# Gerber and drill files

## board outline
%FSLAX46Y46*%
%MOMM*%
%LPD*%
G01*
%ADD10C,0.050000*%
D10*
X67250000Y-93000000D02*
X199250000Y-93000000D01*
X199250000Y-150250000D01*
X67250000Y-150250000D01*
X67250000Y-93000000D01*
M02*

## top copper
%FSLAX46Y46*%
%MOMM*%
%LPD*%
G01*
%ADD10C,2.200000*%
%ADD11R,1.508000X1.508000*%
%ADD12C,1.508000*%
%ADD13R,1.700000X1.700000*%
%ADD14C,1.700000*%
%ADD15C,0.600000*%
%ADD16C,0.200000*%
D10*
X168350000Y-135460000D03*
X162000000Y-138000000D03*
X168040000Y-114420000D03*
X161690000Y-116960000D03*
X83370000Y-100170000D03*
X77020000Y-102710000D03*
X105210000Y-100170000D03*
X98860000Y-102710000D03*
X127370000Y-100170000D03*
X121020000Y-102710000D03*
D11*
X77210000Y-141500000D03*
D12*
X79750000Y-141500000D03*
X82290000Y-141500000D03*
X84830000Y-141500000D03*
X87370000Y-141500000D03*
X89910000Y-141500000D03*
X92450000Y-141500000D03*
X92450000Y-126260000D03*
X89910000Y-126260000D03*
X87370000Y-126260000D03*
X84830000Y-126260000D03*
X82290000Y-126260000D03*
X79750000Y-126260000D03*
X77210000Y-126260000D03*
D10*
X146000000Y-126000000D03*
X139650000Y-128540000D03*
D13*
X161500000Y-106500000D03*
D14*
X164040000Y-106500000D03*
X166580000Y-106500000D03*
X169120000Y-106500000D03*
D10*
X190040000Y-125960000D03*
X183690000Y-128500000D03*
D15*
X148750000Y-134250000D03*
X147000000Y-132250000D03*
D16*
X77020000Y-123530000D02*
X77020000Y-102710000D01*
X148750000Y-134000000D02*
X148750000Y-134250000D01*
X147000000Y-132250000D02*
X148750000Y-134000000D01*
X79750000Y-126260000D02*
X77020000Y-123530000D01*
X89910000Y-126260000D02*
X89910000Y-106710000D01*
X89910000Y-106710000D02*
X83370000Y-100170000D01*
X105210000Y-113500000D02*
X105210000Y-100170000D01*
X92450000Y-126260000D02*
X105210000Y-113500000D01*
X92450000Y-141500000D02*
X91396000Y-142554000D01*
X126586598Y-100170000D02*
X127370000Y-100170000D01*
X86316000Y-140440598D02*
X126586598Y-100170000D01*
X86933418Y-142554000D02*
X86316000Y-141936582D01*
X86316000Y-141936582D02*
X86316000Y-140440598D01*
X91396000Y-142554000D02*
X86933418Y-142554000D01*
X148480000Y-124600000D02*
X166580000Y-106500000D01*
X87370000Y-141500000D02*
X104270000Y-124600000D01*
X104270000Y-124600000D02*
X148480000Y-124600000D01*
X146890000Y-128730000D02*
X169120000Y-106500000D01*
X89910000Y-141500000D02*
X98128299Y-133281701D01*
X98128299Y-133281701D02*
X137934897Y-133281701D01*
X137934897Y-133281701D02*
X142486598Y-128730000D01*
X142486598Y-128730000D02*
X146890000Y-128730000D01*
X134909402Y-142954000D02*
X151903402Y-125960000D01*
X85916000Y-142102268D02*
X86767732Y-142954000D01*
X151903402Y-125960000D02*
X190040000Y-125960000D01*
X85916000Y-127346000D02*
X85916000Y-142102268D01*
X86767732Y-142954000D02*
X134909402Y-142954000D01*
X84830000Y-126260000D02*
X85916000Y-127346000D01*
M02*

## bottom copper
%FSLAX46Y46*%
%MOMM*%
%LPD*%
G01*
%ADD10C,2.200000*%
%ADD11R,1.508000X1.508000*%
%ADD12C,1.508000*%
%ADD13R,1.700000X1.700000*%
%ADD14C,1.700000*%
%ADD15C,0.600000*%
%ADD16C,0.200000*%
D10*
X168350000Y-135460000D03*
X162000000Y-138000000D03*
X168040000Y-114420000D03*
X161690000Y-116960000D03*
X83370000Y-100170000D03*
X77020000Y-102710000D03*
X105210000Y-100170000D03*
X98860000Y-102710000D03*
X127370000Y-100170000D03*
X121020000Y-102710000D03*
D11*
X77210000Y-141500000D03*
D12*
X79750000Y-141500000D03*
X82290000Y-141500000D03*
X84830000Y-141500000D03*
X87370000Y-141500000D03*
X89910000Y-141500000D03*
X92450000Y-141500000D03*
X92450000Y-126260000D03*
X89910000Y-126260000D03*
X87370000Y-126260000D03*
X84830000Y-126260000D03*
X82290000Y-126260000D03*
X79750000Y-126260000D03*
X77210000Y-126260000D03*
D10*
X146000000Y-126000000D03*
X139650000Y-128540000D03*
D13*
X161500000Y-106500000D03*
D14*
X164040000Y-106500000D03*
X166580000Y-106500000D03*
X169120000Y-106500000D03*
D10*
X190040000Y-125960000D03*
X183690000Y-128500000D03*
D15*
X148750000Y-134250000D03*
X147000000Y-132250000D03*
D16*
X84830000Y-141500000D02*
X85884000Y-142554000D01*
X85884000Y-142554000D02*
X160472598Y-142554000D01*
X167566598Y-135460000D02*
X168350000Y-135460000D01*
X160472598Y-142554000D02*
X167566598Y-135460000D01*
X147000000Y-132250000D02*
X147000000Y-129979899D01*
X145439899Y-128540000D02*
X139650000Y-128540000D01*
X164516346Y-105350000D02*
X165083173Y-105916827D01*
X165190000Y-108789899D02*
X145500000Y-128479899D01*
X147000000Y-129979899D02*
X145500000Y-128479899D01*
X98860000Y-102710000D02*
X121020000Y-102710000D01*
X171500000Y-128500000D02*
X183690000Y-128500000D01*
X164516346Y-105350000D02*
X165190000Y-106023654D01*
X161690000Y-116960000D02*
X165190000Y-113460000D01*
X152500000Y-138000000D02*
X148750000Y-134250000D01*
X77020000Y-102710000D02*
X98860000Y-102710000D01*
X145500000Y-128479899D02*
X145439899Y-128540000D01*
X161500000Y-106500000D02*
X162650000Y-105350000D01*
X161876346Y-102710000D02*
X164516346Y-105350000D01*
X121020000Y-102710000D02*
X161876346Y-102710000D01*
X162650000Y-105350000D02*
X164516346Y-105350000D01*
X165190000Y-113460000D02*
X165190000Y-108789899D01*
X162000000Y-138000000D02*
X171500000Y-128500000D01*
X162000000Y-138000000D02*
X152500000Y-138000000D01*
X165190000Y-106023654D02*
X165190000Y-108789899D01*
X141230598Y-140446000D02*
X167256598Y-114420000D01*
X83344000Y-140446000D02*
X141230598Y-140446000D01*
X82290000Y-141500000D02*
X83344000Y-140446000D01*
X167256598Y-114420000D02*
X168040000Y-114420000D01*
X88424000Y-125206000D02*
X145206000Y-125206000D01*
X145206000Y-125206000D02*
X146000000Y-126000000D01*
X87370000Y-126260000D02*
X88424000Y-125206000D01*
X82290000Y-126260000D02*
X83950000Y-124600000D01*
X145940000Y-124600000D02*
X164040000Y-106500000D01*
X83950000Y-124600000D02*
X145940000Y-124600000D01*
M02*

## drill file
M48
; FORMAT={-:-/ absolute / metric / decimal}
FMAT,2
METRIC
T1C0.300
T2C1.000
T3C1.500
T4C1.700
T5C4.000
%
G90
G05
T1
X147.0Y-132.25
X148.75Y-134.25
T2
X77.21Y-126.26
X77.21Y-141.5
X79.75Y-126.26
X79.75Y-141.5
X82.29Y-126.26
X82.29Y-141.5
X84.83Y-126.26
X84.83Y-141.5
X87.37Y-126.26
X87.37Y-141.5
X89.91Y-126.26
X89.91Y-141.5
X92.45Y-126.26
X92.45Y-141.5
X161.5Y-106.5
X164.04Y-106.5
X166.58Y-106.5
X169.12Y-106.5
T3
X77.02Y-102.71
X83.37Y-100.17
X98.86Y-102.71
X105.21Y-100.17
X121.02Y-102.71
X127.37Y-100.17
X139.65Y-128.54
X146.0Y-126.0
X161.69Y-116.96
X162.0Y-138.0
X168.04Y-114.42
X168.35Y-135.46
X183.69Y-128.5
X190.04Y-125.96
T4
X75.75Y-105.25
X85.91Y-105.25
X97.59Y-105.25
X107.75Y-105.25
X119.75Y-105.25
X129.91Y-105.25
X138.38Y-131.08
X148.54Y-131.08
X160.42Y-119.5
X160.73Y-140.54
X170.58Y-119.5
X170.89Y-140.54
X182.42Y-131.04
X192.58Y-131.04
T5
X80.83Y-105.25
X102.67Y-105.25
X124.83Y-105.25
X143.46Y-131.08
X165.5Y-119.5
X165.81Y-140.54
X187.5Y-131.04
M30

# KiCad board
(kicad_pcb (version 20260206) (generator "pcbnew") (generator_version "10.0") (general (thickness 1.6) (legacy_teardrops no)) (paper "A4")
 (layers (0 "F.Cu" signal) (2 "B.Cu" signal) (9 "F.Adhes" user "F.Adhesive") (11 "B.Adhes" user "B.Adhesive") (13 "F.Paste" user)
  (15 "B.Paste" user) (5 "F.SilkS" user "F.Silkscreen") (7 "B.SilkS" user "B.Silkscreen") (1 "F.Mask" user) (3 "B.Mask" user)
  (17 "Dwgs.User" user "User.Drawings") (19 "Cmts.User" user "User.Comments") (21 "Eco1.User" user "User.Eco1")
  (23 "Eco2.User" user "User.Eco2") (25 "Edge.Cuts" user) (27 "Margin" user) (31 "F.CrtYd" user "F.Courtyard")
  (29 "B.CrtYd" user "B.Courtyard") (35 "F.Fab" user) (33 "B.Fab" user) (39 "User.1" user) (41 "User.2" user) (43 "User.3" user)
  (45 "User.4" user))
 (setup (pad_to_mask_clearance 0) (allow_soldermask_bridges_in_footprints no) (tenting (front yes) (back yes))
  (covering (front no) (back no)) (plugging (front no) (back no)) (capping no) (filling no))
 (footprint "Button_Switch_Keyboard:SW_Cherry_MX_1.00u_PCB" (layer "F.Cu") (at 168.35 135.46)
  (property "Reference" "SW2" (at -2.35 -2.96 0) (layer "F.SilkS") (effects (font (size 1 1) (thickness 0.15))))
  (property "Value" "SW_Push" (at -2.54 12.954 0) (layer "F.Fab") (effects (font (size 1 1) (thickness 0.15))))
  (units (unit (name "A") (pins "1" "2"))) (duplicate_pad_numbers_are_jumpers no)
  (pad "" np_thru_hole circle (at -7.62 5.08) (size 1.7 1.7) (drill 1.7) (layers "*.Cu" "*.Mask"))
  (pad "" np_thru_hole circle (at -2.54 5.08) (size 4 4) (drill 4) (layers "*.Cu" "*.Mask"))
  (pad "" np_thru_hole circle (at 2.54 5.08) (size 1.7 1.7) (drill 1.7) (layers "*.Cu" "*.Mask"))
  (pad "1" thru_hole circle (at 0 0) (size 2.2 2.2) (drill 1.5) (layers "*.Cu" "*.Mask") (remove_unused_layers no) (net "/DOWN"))
  (pad "2" thru_hole circle (at -6.35 2.54) (size 2.2 2.2) (drill 1.5) (layers "*.Cu" "*.Mask") (remove_unused_layers no) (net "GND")))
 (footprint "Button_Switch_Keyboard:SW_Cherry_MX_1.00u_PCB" (layer "F.Cu") (at 168.04 114.42)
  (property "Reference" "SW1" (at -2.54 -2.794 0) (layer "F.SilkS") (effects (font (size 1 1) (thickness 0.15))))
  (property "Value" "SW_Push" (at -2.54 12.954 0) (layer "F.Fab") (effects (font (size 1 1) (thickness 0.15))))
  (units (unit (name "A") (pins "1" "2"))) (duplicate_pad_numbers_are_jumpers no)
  (pad "" np_thru_hole circle (at -7.62 5.08) (size 1.7 1.7) (drill 1.7) (layers "*.Cu" "*.Mask"))
  (pad "" np_thru_hole circle (at -2.54 5.08) (size 4 4) (drill 4) (layers "*.Cu" "*.Mask"))
  (pad "" np_thru_hole circle (at 2.54 5.08) (size 1.7 1.7) (drill 1.7) (layers "*.Cu" "*.Mask"))
  (pad "1" thru_hole circle (at 0 0) (size 2.2 2.2) (drill 1.5) (layers "*.Cu" "*.Mask") (remove_unused_layers no) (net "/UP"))
  (pad "2" thru_hole circle (at -6.35 2.54) (size 2.2 2.2) (drill 1.5) (layers "*.Cu" "*.Mask") (remove_unused_layers no) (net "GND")))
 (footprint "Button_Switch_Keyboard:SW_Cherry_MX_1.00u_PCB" (layer "F.Cu") (at 83.37 100.17)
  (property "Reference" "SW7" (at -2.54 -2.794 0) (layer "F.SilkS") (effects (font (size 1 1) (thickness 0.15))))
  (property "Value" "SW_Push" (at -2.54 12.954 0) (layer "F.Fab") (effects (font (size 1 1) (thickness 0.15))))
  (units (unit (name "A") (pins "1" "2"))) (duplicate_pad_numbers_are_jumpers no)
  (pad "" np_thru_hole circle (at -7.62 5.08) (size 1.7 1.7) (drill 1.7) (layers "*.Cu" "*.Mask"))
  (pad "" np_thru_hole circle (at -2.54 5.08) (size 4 4) (drill 4) (layers "*.Cu" "*.Mask"))
  (pad "" np_thru_hole circle (at 2.54 5.08) (size 1.7 1.7) (drill 1.7) (layers "*.Cu" "*.Mask"))
  (pad "1" thru_hole circle (at 0 0) (size 2.2 2.2) (drill 1.5) (layers "*.Cu" "*.Mask") (remove_unused_layers no) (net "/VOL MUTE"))
  (pad "2" thru_hole circle (at -6.35 2.54) (size 2.2 2.2) (drill 1.5) (layers "*.Cu" "*.Mask") (remove_unused_layers no) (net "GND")))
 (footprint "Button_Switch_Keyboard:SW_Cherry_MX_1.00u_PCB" (layer "F.Cu") (at 105.21 100.17)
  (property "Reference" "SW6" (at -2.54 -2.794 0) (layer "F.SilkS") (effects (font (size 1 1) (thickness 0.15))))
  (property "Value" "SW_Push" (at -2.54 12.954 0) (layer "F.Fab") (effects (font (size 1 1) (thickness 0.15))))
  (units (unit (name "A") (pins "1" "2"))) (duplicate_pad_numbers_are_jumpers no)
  (pad "" np_thru_hole circle (at -7.62 5.08) (size 1.7 1.7) (drill 1.7) (layers "*.Cu" "*.Mask"))
  (pad "" np_thru_hole circle (at -2.54 5.08) (size 4 4) (drill 4) (layers "*.Cu" "*.Mask"))
  (pad "" np_thru_hole circle (at 2.54 5.08) (size 1.7 1.7) (drill 1.7) (layers "*.Cu" "*.Mask"))
  (pad "1" thru_hole circle (at 0 0) (size 2.2 2.2) (drill 1.5) (layers "*.Cu" "*.Mask") (remove_unused_layers no) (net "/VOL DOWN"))
  (pad "2" thru_hole circle (at -6.35 2.54) (size 2.2 2.2) (drill 1.5) (layers "*.Cu" "*.Mask") (remove_unused_layers no) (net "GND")))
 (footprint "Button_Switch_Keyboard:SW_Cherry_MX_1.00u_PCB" (layer "F.Cu") (at 127.37 100.17)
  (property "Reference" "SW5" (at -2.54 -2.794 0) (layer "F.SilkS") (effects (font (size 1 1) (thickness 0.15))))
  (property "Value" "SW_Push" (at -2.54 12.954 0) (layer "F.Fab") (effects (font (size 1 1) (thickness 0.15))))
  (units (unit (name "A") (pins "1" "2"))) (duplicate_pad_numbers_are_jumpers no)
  (pad "" np_thru_hole circle (at -7.62 5.08) (size 1.7 1.7) (drill 1.7) (layers "*.Cu" "*.Mask"))
  (pad "" np_thru_hole circle (at -2.54 5.08) (size 4 4) (drill 4) (layers "*.Cu" "*.Mask"))
  (pad "" np_thru_hole circle (at 2.54 5.08) (size 1.7 1.7) (drill 1.7) (layers "*.Cu" "*.Mask"))
  (pad "1" thru_hole circle (at 0 0) (size 2.2 2.2) (drill 1.5) (layers "*.Cu" "*.Mask") (remove_unused_layers no) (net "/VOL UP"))
  (pad "2" thru_hole circle (at -6.35 2.54) (size 2.2 2.2) (drill 1.5) (layers "*.Cu" "*.Mask") (remove_unused_layers no) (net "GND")))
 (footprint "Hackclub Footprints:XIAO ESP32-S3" (layer "F.Cu") (at 84.7665 133.88 90)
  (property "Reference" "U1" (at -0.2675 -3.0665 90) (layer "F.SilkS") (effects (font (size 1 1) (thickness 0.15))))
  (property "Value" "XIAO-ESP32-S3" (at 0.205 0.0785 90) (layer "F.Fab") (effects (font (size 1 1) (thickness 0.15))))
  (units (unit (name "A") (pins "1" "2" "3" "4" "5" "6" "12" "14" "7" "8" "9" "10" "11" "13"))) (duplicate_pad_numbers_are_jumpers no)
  (pad "1" thru_hole rect (at -7.62 -7.5565 90) (size 1.508 1.508) (drill 1) (layers "*.Cu" "*.Mask") (remove_unused_layers no)
   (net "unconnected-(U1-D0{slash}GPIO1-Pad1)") (solder_mask_margin 0.102))
  (pad "2" thru_hole circle (at -7.62 -5.0165 90) (size 1.508 1.508) (drill 1) (layers "*.Cu" "*.Mask") (remove_unused_layers no)
   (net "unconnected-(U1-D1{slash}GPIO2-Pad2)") (solder_mask_margin 0.102))
  (pad "3" thru_hole circle (at -7.62 -2.4765 90) (size 1.508 1.508) (drill 1) (layers "*.Cu" "*.Mask") (remove_unused_layers no)
   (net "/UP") (solder_mask_margin 0.102))
  (pad "4" thru_hole circle (at -7.62 0.0635 90) (size 1.508 1.508) (drill 1) (layers "*.Cu" "*.Mask") (remove_unused_layers no)
   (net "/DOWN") (solder_mask_margin 0.102))
  (pad "5" thru_hole circle (at -7.62 2.6035 90) (size 1.508 1.508) (drill 1) (layers "*.Cu" "*.Mask") (remove_unused_layers no)
   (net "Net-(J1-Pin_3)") (solder_mask_margin 0.102))
  (pad "6" thru_hole circle (at -7.62 5.1435 90) (size 1.508 1.508) (drill 1) (layers "*.Cu" "*.Mask") (remove_unused_layers no)
   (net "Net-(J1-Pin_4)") (solder_mask_margin 0.102))
  (pad "7" thru_hole circle (at -7.62 7.6835 90) (size 1.508 1.508) (drill 1) (layers "*.Cu" "*.Mask") (remove_unused_layers no)
   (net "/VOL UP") (solder_mask_margin 0.102))
  (pad "8" thru_hole circle (at 7.62 7.6835 90) (size 1.508 1.508) (drill 1) (layers "*.Cu" "*.Mask") (remove_unused_layers no)
   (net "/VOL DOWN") (solder_mask_margin 0.102))
  (pad "9" thru_hole circle (at 7.62 5.1435 90) (size 1.508 1.508) (drill 1) (layers "*.Cu" "*.Mask") (remove_unused_layers no)
   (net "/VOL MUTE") (solder_mask_margin 0.102))
  (pad "10" thru_hole circle (at 7.62 2.6035 90) (size 1.508 1.508) (drill 1) (layers "*.Cu" "*.Mask") (remove_unused_layers no)
   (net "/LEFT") (solder_mask_margin 0.102))
  (pad "11" thru_hole circle (at 7.62 0.0635 90) (size 1.508 1.508) (drill 1) (layers "*.Cu" "*.Mask") (remove_unused_layers no)
   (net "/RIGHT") (solder_mask_margin 0.102))
  (pad "12" thru_hole circle (at 7.62 -2.4765 90) (size 1.508 1.508) (drill 1) (layers "*.Cu" "*.Mask") (remove_unused_layers no)
   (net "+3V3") (solder_mask_margin 0.102))
  (pad "13" thru_hole circle (at 7.62 -5.0165 90) (size 1.508 1.508) (drill 1) (layers "*.Cu" "*.Mask") (remove_unused_layers no)
   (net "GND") (solder_mask_margin 0.102))
  (pad "14" thru_hole circle (at 7.62 -7.5565 90) (size 1.508 1.508) (drill 1) (layers "*.Cu" "*.Mask") (remove_unused_layers no)
   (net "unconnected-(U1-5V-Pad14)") (solder_mask_margin 0.102)))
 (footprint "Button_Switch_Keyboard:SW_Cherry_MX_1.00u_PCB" (layer "F.Cu") (at 146 126)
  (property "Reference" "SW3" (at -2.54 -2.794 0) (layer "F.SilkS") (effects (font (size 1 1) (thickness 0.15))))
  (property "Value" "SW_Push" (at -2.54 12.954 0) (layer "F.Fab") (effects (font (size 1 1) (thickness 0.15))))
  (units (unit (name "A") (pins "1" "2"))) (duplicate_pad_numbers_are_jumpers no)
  (pad "" np_thru_hole circle (at -7.62 5.08) (size 1.7 1.7) (drill 1.7) (layers "*.Cu" "*.Mask"))
  (pad "" np_thru_hole circle (at -2.54 5.08) (size 4 4) (drill 4) (layers "*.Cu" "*.Mask"))
  (pad "" np_thru_hole circle (at 2.54 5.08) (size 1.7 1.7) (drill 1.7) (layers "*.Cu" "*.Mask"))
  (pad "1" thru_hole circle (at 0 0) (size 2.2 2.2) (drill 1.5) (layers "*.Cu" "*.Mask") (remove_unused_layers no) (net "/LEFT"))
  (pad "2" thru_hole circle (at -6.35 2.54) (size 2.2 2.2) (drill 1.5) (layers "*.Cu" "*.Mask") (remove_unused_layers no) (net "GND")))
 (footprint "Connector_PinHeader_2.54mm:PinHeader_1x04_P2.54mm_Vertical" (layer "F.Cu") (at 161.5 106.5 90)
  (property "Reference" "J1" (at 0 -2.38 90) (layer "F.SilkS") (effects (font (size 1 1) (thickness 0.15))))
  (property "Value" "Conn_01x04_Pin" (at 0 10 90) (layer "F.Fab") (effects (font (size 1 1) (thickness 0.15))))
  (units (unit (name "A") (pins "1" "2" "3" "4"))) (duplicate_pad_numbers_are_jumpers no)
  (pad "1" thru_hole rect (at 0 0 90) (size 1.7 1.7) (drill 1) (layers "*.Cu" "*.Mask") (remove_unused_layers no) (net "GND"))
  (pad "2" thru_hole circle (at 0 2.54 90) (size 1.7 1.7) (drill 1) (layers "*.Cu" "*.Mask") (remove_unused_layers no) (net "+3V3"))
  (pad "3" thru_hole circle (at 0 5.08 90) (size 1.7 1.7) (drill 1) (layers "*.Cu" "*.Mask") (remove_unused_layers no)
   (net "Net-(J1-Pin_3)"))
  (pad "4" thru_hole circle (at 0 7.62 90) (size 1.7 1.7) (drill 1) (layers "*.Cu" "*.Mask") (remove_unused_layers no)
   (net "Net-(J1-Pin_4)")))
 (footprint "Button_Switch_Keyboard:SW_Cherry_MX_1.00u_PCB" (layer "F.Cu") (at 190.04 125.96)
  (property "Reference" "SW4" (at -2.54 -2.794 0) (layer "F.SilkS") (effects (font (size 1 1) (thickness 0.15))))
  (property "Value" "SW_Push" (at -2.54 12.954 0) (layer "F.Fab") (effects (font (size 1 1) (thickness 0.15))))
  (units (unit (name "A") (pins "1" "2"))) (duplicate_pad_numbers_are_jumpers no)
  (pad "" np_thru_hole circle (at -7.62 5.08) (size 1.7 1.7) (drill 1.7) (layers "*.Cu" "*.Mask"))
  (pad "" np_thru_hole circle (at -2.54 5.08) (size 4 4) (drill 4) (layers "*.Cu" "*.Mask"))
  (pad "" np_thru_hole circle (at 2.54 5.08) (size 1.7 1.7) (drill 1.7) (layers "*.Cu" "*.Mask"))
  (pad "1" thru_hole circle (at 0 0) (size 2.2 2.2) (drill 1.5) (layers "*.Cu" "*.Mask") (remove_unused_layers no) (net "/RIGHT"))
  (pad "2" thru_hole circle (at -6.35 2.54) (size 2.2 2.2) (drill 1.5) (layers "*.Cu" "*.Mask") (remove_unused_layers no) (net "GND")))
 (gr_rect (start 67.25 93) (end 199.25 150.25) (stroke (width 0.05) (type default)) (fill no) (layer "Edge.Cuts"))
 (segment (start 84.83 141.5) (end 85.884 142.554) (width 0.2) (layer "B.Cu") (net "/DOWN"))
 (segment (start 85.884 142.554) (end 160.472598 142.554) (width 0.2) (layer "B.Cu") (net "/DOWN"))
 (segment (start 167.566598 135.46) (end 168.35 135.46) (width 0.2) (layer "B.Cu") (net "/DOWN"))
 (segment (start 160.472598 142.554) (end 167.566598 135.46) (width 0.2) (layer "B.Cu") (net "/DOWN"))
 (segment (start 77.02 123.53) (end 77.02 102.71) (width 0.2) (layer "F.Cu") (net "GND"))
 (segment (start 148.75 134) (end 148.75 134.25) (width 0.2) (layer "F.Cu") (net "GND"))
 (segment (start 147 132.25) (end 148.75 134) (width 0.2) (layer "F.Cu") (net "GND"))
 (segment (start 79.75 126.26) (end 77.02 123.53) (width 0.2) (layer "F.Cu") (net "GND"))
 (via (at 148.75 134.25) (size 0.6) (drill 0.3) (layers "F.Cu" "B.Cu") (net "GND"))
 (via (at 147 132.25) (size 0.6) (drill 0.3) (layers "F.Cu" "B.Cu") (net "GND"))
 (segment (start 147 132.25) (end 147 129.979899) (width 0.2) (layer "B.Cu") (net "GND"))
 (segment (start 145.439899 128.54) (end 139.65 128.54) (width 0.2) (layer "B.Cu") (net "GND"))
 (segment (start 164.516346 105.35) (end 165.083173 105.916827) (width 0.2) (layer "B.Cu") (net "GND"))
 (segment (start 165.19 108.789899) (end 145.5 128.479899) (width 0.2) (layer "B.Cu") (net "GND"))
 (segment (start 147 129.979899) (end 145.5 128.479899) (width 0.2) (layer "B.Cu") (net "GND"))
 (segment (start 98.86 102.71) (end 121.02 102.71) (width 0.2) (layer "B.Cu") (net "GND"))
 (segment (start 171.5 128.5) (end 183.69 128.5) (width 0.2) (layer "B.Cu") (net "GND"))
 (segment (start 164.516346 105.35) (end 165.19 106.023654) (width 0.2) (layer "B.Cu") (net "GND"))
 (segment (start 161.69 116.96) (end 165.19 113.46) (width 0.2) (layer "B.Cu") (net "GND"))
 (segment (start 152.5 138) (end 148.75 134.25) (width 0.2) (layer "B.Cu") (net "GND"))
 (segment (start 77.02 102.71) (end 98.86 102.71) (width 0.2) (layer "B.Cu") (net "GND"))
 (segment (start 145.5 128.479899) (end 145.439899 128.54) (width 0.2) (layer "B.Cu") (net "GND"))
 (segment (start 161.5 106.5) (end 162.65 105.35) (width 0.2) (layer "B.Cu") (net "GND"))
 (segment (start 161.876346 102.71) (end 164.516346 105.35) (width 0.2) (layer "B.Cu") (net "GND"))
 (segment (start 121.02 102.71) (end 161.876346 102.71) (width 0.2) (layer "B.Cu") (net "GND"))
 (segment (start 162.65 105.35) (end 164.516346 105.35) (width 0.2) (layer "B.Cu") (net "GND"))
 (segment (start 165.19 113.46) (end 165.19 108.789899) (width 0.2) (layer "B.Cu") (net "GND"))
 (segment (start 162 138) (end 171.5 128.5) (width 0.2) (layer "B.Cu") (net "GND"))
 (segment (start 162 138) (end 152.5 138) (width 0.2) (layer "B.Cu") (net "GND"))
 (segment (start 165.19 106.023654) (end 165.19 108.789899) (width 0.2) (layer "B.Cu") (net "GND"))
 (segment (start 141.230598 140.446) (end 167.256598 114.42) (width 0.2) (layer "B.Cu") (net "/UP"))
 (segment (start 83.344 140.446) (end 141.230598 140.446) (width 0.2) (layer "B.Cu") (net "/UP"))
 (segment (start 82.29 141.5) (end 83.344 140.446) (width 0.2) (layer "B.Cu") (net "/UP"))
 (segment (start 167.256598 114.42) (end 168.04 114.42) (width 0.2) (layer "B.Cu") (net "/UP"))
 (segment (start 89.91 126.26) (end 89.91 106.71) (width 0.2) (layer "F.Cu") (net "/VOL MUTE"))
 (segment (start 89.91 106.71) (end 83.37 100.17) (width 0.2) (layer "F.Cu") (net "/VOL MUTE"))
 (segment (start 105.21 113.5) (end 105.21 100.17) (width 0.2) (layer "F.Cu") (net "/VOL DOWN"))
 (segment (start 92.45 126.26) (end 105.21 113.5) (width 0.2) (layer "F.Cu") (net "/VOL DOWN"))
 (segment (start 92.45 141.5) (end 91.396 142.554) (width 0.2) (layer "F.Cu") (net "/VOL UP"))
 (segment (start 126.586598 100.17) (end 127.37 100.17) (width 0.2) (layer "F.Cu") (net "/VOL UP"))
 (segment (start 86.316 140.440598) (end 126.586598 100.17) (width 0.2) (layer "F.Cu") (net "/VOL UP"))
 (segment (start 86.933418 142.554) (end 86.316 141.936582) (width 0.2) (layer "F.Cu") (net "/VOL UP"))
 (segment (start 86.316 141.936582) (end 86.316 140.440598) (width 0.2) (layer "F.Cu") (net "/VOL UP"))
 (segment (start 91.396 142.554) (end 86.933418 142.554) (width 0.2) (layer "F.Cu") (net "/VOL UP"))
 (segment (start 148.48 124.6) (end 166.58 106.5) (width 0.2) (layer "F.Cu") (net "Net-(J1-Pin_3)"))
 (segment (start 87.37 141.5) (end 104.27 124.6) (width 0.2) (layer "F.Cu") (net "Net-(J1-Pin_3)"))
 (segment (start 104.27 124.6) (end 148.48 124.6) (width 0.2) (layer "F.Cu") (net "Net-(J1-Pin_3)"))
 (segment (start 146.89 128.73) (end 169.12 106.5) (width 0.2) (layer "F.Cu") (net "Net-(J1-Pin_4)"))
 (segment (start 89.91 141.5) (end 98.128299 133.281701) (width 0.2) (layer "F.Cu") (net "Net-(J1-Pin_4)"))
 (segment (start 98.128299 133.281701) (end 137.934897 133.281701) (width 0.2) (layer "F.Cu") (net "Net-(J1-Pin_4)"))
 (segment (start 137.934897 133.281701) (end 142.486598 128.73) (width 0.2) (layer "F.Cu") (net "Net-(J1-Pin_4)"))
 (segment (start 142.486598 128.73) (end 146.89 128.73) (width 0.2) (layer "F.Cu") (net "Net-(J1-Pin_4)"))
 (segment (start 88.424 125.206) (end 145.206 125.206) (width 0.2) (layer "B.Cu") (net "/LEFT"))
 (segment (start 145.206 125.206) (end 146 126) (width 0.2) (layer "B.Cu") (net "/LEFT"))
 (segment (start 87.37 126.26) (end 88.424 125.206) (width 0.2) (layer "B.Cu") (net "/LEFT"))
 (segment (start 134.909402 142.954) (end 151.903402 125.96) (width 0.2) (layer "F.Cu") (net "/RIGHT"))
 (segment (start 85.916 142.102268) (end 86.767732 142.954) (width 0.2) (layer "F.Cu") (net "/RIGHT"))
 (segment (start 151.903402 125.96) (end 190.04 125.96) (width 0.2) (layer "F.Cu") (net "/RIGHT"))
 (segment (start 85.916 127.346) (end 85.916 142.102268) (width 0.2) (layer "F.Cu") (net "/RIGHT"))
 (segment (start 86.767732 142.954) (end 134.909402 142.954) (width 0.2) (layer "F.Cu") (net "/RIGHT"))
 (segment (start 84.83 126.26) (end 85.916 127.346) (width 0.2) (layer "F.Cu") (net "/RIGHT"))
 (segment (start 82.29 126.26) (end 83.95 124.6) (width 0.2) (layer "B.Cu") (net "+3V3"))
 (segment (start 145.94 124.6) (end 164.04 106.5) (width 0.2) (layer "B.Cu") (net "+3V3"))
 (segment (start 83.95 124.6) (end 145.94 124.6) (width 0.2) (layer "B.Cu") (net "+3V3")))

